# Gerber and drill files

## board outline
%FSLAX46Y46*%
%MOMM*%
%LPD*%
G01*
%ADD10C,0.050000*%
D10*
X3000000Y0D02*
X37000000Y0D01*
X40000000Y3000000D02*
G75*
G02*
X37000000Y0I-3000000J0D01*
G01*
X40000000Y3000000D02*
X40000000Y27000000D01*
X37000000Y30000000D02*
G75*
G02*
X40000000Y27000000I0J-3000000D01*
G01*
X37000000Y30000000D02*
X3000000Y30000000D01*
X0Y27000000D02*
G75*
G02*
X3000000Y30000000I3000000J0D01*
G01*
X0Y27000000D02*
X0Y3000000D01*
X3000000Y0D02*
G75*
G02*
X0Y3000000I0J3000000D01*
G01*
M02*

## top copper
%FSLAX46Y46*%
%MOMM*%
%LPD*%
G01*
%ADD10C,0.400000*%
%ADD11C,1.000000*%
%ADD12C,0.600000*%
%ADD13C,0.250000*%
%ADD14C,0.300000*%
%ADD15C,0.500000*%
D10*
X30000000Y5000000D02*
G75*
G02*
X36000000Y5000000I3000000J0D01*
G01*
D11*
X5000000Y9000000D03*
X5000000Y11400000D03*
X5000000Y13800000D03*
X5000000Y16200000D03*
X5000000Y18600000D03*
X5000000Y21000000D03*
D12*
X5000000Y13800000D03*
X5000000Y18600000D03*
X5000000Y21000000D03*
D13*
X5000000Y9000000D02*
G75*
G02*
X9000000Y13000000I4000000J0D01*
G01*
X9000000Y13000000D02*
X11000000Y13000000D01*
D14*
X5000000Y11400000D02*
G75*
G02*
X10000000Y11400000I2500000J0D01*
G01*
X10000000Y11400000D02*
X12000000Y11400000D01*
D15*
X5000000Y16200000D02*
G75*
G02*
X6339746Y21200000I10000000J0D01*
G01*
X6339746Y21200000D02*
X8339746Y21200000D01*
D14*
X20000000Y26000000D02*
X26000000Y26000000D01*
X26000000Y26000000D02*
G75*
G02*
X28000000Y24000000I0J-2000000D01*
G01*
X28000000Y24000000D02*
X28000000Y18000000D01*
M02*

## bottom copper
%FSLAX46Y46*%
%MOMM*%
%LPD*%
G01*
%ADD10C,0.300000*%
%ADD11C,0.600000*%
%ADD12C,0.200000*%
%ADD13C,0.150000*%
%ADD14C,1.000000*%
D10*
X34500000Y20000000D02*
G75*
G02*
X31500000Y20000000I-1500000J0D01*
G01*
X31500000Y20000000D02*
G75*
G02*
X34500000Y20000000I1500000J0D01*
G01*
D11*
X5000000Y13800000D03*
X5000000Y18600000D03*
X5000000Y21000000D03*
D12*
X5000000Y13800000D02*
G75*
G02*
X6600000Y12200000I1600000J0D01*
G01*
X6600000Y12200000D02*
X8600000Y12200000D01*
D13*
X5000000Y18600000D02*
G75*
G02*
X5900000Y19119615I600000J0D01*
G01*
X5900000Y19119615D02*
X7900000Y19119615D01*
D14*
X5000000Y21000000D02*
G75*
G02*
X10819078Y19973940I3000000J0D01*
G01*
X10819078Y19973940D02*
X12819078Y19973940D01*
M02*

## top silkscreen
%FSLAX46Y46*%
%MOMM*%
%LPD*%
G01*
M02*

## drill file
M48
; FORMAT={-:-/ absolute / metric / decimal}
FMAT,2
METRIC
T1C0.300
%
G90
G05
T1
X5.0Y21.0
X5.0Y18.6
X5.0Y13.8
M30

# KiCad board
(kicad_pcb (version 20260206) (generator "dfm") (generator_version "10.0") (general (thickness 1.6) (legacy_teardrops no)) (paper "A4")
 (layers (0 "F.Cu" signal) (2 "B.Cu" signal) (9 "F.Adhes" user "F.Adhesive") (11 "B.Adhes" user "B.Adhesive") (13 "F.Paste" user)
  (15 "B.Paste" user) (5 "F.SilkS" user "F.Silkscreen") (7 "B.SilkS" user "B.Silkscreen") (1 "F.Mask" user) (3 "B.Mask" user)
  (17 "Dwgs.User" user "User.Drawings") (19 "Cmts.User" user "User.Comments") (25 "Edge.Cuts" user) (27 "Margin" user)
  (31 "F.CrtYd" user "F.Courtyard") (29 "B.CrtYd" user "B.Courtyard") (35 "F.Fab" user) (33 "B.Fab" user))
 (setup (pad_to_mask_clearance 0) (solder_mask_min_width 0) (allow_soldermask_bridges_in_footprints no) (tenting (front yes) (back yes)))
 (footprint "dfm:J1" (layer "F.Cu") (at 5 -15 0)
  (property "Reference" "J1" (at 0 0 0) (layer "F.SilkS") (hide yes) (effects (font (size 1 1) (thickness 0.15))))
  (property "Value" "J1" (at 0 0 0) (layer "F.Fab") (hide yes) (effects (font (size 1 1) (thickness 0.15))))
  (pad "1" smd circle (at 0 6 0) (size 1 1) (layers "F.Cu" "F.Mask" "F.Paste") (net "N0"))
  (pad "2" smd circle (at 0 3.6 0) (size 1 1) (layers "F.Cu" "F.Mask" "F.Paste") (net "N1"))
  (pad "3" smd circle (at 0 1.2 0) (size 1 1) (layers "F.Cu" "F.Mask" "F.Paste") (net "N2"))
  (pad "4" smd circle (at 0 -1.2 0) (size 1 1) (layers "F.Cu" "F.Mask" "F.Paste") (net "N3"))
  (pad "5" smd circle (at 0 -3.6 0) (size 1 1) (layers "F.Cu" "F.Mask" "F.Paste") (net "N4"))
  (pad "6" smd circle (at 0 -6 0) (size 1 1) (layers "F.Cu" "F.Mask" "F.Paste") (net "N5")))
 (gr_line (start 3 0) (end 37 0) (stroke (width 0.05) (type solid)) (layer "Edge.Cuts"))
 (gr_arc (start 37 0) (mid 39.12132 -0.87868) (end 40 -3) (stroke (width 0.05) (type solid)) (layer "Edge.Cuts"))
 (gr_line (start 40 -3) (end 40 -27) (stroke (width 0.05) (type solid)) (layer "Edge.Cuts"))
 (gr_arc (start 40 -27) (mid 39.12132 -29.12132) (end 37 -30) (stroke (width 0.05) (type solid)) (layer "Edge.Cuts"))
 (gr_line (start 37 -30) (end 3 -30) (stroke (width 0.05) (type solid)) (layer "Edge.Cuts"))
 (gr_arc (start 3 -30) (mid 0.87868 -29.12132) (end 0 -27) (stroke (width 0.05) (type solid)) (layer "Edge.Cuts"))
 (gr_line (start 0 -27) (end 0 -3) (stroke (width 0.05) (type solid)) (layer "Edge.Cuts"))
 (gr_arc (start 0 -3) (mid 0.87868 -0.87868) (end 3 0) (stroke (width 0.05) (type solid)) (layer "Edge.Cuts"))
 (arc (start 5 -9) (mid 6.171573 -11.828427) (end 9 -13) (width 0.25) (layer "F.Cu") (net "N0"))
 (segment (start 9 -13) (end 11 -13) (width 0.25) (layer "F.Cu") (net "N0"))
 (arc (start 5 -11.4) (mid 7.5 -13.9) (end 10 -11.4) (width 0.3) (layer "F.Cu") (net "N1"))
 (segment (start 10 -11.4) (end 12 -11.4) (width 0.3) (layer "F.Cu") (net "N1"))
 (via (at 5 -13.8) (size 0.6) (drill 0.3) (layers "F.Cu" "B.Cu") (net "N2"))
 (arc (start 5 -13.8) (mid 7.731371 -14.931371) (end 6.6 -12.2) (width 0.2) (layer "B.Cu") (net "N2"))
 (segment (start 6.6 -12.2) (end 8.6 -12.2) (width 0.2) (layer "B.Cu") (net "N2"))
 (arc (start 5 -16.2) (mid 5.340742 -18.78819) (end 6.339746 -21.2) (width 0.5) (layer "F.Cu") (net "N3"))
 (segment (start 6.339746 -21.2) (end 8.339746 -21.2) (width 0.5) (layer "F.Cu") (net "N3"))
 (via (at 5 -18.6) (size 0.6) (drill 0.3) (layers "F.Cu" "B.Cu") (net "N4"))
 (arc (start 5 -18.6) (mid 5.3 -19.119615) (end 5.9 -19.119615) (width 0.15) (layer "B.Cu") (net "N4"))
 (segment (start 5.9 -19.119615) (end 7.9 -19.119615) (width 0.15) (layer "B.Cu") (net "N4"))
 (via (at 5 -21) (size 0.6) (drill 0.3) (layers "F.Cu" "B.Cu") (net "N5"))
 (arc (start 5 -21) (mid 8.520945 -23.954423) (end 10.819078 -19.97394) (width 1) (layer "B.Cu") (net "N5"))
 (segment (start 10.819078 -19.97394) (end 12.819078 -19.97394) (width 1) (layer "B.Cu") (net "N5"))
 (segment (start 20 -26) (end 26 -26) (width 0.3) (layer "F.Cu") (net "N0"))
 (arc (start 26 -26) (mid 27.414214 -25.414214) (end 28 -24) (width 0.3) (layer "F.Cu") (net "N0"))
 (segment (start 28 -24) (end 28 -18) (width 0.3) (layer "F.Cu") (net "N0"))
 (gr_arc (start 30 -5) (mid 33 -8) (end 36 -5) (stroke (width 0.4) (type solid)) (layer "F.Cu") (net "N1"))
 (gr_circle (center 33 -20) (end 34.5 -20) (stroke (width 0.3) (type solid)) (fill no) (layer "B.Cu")))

